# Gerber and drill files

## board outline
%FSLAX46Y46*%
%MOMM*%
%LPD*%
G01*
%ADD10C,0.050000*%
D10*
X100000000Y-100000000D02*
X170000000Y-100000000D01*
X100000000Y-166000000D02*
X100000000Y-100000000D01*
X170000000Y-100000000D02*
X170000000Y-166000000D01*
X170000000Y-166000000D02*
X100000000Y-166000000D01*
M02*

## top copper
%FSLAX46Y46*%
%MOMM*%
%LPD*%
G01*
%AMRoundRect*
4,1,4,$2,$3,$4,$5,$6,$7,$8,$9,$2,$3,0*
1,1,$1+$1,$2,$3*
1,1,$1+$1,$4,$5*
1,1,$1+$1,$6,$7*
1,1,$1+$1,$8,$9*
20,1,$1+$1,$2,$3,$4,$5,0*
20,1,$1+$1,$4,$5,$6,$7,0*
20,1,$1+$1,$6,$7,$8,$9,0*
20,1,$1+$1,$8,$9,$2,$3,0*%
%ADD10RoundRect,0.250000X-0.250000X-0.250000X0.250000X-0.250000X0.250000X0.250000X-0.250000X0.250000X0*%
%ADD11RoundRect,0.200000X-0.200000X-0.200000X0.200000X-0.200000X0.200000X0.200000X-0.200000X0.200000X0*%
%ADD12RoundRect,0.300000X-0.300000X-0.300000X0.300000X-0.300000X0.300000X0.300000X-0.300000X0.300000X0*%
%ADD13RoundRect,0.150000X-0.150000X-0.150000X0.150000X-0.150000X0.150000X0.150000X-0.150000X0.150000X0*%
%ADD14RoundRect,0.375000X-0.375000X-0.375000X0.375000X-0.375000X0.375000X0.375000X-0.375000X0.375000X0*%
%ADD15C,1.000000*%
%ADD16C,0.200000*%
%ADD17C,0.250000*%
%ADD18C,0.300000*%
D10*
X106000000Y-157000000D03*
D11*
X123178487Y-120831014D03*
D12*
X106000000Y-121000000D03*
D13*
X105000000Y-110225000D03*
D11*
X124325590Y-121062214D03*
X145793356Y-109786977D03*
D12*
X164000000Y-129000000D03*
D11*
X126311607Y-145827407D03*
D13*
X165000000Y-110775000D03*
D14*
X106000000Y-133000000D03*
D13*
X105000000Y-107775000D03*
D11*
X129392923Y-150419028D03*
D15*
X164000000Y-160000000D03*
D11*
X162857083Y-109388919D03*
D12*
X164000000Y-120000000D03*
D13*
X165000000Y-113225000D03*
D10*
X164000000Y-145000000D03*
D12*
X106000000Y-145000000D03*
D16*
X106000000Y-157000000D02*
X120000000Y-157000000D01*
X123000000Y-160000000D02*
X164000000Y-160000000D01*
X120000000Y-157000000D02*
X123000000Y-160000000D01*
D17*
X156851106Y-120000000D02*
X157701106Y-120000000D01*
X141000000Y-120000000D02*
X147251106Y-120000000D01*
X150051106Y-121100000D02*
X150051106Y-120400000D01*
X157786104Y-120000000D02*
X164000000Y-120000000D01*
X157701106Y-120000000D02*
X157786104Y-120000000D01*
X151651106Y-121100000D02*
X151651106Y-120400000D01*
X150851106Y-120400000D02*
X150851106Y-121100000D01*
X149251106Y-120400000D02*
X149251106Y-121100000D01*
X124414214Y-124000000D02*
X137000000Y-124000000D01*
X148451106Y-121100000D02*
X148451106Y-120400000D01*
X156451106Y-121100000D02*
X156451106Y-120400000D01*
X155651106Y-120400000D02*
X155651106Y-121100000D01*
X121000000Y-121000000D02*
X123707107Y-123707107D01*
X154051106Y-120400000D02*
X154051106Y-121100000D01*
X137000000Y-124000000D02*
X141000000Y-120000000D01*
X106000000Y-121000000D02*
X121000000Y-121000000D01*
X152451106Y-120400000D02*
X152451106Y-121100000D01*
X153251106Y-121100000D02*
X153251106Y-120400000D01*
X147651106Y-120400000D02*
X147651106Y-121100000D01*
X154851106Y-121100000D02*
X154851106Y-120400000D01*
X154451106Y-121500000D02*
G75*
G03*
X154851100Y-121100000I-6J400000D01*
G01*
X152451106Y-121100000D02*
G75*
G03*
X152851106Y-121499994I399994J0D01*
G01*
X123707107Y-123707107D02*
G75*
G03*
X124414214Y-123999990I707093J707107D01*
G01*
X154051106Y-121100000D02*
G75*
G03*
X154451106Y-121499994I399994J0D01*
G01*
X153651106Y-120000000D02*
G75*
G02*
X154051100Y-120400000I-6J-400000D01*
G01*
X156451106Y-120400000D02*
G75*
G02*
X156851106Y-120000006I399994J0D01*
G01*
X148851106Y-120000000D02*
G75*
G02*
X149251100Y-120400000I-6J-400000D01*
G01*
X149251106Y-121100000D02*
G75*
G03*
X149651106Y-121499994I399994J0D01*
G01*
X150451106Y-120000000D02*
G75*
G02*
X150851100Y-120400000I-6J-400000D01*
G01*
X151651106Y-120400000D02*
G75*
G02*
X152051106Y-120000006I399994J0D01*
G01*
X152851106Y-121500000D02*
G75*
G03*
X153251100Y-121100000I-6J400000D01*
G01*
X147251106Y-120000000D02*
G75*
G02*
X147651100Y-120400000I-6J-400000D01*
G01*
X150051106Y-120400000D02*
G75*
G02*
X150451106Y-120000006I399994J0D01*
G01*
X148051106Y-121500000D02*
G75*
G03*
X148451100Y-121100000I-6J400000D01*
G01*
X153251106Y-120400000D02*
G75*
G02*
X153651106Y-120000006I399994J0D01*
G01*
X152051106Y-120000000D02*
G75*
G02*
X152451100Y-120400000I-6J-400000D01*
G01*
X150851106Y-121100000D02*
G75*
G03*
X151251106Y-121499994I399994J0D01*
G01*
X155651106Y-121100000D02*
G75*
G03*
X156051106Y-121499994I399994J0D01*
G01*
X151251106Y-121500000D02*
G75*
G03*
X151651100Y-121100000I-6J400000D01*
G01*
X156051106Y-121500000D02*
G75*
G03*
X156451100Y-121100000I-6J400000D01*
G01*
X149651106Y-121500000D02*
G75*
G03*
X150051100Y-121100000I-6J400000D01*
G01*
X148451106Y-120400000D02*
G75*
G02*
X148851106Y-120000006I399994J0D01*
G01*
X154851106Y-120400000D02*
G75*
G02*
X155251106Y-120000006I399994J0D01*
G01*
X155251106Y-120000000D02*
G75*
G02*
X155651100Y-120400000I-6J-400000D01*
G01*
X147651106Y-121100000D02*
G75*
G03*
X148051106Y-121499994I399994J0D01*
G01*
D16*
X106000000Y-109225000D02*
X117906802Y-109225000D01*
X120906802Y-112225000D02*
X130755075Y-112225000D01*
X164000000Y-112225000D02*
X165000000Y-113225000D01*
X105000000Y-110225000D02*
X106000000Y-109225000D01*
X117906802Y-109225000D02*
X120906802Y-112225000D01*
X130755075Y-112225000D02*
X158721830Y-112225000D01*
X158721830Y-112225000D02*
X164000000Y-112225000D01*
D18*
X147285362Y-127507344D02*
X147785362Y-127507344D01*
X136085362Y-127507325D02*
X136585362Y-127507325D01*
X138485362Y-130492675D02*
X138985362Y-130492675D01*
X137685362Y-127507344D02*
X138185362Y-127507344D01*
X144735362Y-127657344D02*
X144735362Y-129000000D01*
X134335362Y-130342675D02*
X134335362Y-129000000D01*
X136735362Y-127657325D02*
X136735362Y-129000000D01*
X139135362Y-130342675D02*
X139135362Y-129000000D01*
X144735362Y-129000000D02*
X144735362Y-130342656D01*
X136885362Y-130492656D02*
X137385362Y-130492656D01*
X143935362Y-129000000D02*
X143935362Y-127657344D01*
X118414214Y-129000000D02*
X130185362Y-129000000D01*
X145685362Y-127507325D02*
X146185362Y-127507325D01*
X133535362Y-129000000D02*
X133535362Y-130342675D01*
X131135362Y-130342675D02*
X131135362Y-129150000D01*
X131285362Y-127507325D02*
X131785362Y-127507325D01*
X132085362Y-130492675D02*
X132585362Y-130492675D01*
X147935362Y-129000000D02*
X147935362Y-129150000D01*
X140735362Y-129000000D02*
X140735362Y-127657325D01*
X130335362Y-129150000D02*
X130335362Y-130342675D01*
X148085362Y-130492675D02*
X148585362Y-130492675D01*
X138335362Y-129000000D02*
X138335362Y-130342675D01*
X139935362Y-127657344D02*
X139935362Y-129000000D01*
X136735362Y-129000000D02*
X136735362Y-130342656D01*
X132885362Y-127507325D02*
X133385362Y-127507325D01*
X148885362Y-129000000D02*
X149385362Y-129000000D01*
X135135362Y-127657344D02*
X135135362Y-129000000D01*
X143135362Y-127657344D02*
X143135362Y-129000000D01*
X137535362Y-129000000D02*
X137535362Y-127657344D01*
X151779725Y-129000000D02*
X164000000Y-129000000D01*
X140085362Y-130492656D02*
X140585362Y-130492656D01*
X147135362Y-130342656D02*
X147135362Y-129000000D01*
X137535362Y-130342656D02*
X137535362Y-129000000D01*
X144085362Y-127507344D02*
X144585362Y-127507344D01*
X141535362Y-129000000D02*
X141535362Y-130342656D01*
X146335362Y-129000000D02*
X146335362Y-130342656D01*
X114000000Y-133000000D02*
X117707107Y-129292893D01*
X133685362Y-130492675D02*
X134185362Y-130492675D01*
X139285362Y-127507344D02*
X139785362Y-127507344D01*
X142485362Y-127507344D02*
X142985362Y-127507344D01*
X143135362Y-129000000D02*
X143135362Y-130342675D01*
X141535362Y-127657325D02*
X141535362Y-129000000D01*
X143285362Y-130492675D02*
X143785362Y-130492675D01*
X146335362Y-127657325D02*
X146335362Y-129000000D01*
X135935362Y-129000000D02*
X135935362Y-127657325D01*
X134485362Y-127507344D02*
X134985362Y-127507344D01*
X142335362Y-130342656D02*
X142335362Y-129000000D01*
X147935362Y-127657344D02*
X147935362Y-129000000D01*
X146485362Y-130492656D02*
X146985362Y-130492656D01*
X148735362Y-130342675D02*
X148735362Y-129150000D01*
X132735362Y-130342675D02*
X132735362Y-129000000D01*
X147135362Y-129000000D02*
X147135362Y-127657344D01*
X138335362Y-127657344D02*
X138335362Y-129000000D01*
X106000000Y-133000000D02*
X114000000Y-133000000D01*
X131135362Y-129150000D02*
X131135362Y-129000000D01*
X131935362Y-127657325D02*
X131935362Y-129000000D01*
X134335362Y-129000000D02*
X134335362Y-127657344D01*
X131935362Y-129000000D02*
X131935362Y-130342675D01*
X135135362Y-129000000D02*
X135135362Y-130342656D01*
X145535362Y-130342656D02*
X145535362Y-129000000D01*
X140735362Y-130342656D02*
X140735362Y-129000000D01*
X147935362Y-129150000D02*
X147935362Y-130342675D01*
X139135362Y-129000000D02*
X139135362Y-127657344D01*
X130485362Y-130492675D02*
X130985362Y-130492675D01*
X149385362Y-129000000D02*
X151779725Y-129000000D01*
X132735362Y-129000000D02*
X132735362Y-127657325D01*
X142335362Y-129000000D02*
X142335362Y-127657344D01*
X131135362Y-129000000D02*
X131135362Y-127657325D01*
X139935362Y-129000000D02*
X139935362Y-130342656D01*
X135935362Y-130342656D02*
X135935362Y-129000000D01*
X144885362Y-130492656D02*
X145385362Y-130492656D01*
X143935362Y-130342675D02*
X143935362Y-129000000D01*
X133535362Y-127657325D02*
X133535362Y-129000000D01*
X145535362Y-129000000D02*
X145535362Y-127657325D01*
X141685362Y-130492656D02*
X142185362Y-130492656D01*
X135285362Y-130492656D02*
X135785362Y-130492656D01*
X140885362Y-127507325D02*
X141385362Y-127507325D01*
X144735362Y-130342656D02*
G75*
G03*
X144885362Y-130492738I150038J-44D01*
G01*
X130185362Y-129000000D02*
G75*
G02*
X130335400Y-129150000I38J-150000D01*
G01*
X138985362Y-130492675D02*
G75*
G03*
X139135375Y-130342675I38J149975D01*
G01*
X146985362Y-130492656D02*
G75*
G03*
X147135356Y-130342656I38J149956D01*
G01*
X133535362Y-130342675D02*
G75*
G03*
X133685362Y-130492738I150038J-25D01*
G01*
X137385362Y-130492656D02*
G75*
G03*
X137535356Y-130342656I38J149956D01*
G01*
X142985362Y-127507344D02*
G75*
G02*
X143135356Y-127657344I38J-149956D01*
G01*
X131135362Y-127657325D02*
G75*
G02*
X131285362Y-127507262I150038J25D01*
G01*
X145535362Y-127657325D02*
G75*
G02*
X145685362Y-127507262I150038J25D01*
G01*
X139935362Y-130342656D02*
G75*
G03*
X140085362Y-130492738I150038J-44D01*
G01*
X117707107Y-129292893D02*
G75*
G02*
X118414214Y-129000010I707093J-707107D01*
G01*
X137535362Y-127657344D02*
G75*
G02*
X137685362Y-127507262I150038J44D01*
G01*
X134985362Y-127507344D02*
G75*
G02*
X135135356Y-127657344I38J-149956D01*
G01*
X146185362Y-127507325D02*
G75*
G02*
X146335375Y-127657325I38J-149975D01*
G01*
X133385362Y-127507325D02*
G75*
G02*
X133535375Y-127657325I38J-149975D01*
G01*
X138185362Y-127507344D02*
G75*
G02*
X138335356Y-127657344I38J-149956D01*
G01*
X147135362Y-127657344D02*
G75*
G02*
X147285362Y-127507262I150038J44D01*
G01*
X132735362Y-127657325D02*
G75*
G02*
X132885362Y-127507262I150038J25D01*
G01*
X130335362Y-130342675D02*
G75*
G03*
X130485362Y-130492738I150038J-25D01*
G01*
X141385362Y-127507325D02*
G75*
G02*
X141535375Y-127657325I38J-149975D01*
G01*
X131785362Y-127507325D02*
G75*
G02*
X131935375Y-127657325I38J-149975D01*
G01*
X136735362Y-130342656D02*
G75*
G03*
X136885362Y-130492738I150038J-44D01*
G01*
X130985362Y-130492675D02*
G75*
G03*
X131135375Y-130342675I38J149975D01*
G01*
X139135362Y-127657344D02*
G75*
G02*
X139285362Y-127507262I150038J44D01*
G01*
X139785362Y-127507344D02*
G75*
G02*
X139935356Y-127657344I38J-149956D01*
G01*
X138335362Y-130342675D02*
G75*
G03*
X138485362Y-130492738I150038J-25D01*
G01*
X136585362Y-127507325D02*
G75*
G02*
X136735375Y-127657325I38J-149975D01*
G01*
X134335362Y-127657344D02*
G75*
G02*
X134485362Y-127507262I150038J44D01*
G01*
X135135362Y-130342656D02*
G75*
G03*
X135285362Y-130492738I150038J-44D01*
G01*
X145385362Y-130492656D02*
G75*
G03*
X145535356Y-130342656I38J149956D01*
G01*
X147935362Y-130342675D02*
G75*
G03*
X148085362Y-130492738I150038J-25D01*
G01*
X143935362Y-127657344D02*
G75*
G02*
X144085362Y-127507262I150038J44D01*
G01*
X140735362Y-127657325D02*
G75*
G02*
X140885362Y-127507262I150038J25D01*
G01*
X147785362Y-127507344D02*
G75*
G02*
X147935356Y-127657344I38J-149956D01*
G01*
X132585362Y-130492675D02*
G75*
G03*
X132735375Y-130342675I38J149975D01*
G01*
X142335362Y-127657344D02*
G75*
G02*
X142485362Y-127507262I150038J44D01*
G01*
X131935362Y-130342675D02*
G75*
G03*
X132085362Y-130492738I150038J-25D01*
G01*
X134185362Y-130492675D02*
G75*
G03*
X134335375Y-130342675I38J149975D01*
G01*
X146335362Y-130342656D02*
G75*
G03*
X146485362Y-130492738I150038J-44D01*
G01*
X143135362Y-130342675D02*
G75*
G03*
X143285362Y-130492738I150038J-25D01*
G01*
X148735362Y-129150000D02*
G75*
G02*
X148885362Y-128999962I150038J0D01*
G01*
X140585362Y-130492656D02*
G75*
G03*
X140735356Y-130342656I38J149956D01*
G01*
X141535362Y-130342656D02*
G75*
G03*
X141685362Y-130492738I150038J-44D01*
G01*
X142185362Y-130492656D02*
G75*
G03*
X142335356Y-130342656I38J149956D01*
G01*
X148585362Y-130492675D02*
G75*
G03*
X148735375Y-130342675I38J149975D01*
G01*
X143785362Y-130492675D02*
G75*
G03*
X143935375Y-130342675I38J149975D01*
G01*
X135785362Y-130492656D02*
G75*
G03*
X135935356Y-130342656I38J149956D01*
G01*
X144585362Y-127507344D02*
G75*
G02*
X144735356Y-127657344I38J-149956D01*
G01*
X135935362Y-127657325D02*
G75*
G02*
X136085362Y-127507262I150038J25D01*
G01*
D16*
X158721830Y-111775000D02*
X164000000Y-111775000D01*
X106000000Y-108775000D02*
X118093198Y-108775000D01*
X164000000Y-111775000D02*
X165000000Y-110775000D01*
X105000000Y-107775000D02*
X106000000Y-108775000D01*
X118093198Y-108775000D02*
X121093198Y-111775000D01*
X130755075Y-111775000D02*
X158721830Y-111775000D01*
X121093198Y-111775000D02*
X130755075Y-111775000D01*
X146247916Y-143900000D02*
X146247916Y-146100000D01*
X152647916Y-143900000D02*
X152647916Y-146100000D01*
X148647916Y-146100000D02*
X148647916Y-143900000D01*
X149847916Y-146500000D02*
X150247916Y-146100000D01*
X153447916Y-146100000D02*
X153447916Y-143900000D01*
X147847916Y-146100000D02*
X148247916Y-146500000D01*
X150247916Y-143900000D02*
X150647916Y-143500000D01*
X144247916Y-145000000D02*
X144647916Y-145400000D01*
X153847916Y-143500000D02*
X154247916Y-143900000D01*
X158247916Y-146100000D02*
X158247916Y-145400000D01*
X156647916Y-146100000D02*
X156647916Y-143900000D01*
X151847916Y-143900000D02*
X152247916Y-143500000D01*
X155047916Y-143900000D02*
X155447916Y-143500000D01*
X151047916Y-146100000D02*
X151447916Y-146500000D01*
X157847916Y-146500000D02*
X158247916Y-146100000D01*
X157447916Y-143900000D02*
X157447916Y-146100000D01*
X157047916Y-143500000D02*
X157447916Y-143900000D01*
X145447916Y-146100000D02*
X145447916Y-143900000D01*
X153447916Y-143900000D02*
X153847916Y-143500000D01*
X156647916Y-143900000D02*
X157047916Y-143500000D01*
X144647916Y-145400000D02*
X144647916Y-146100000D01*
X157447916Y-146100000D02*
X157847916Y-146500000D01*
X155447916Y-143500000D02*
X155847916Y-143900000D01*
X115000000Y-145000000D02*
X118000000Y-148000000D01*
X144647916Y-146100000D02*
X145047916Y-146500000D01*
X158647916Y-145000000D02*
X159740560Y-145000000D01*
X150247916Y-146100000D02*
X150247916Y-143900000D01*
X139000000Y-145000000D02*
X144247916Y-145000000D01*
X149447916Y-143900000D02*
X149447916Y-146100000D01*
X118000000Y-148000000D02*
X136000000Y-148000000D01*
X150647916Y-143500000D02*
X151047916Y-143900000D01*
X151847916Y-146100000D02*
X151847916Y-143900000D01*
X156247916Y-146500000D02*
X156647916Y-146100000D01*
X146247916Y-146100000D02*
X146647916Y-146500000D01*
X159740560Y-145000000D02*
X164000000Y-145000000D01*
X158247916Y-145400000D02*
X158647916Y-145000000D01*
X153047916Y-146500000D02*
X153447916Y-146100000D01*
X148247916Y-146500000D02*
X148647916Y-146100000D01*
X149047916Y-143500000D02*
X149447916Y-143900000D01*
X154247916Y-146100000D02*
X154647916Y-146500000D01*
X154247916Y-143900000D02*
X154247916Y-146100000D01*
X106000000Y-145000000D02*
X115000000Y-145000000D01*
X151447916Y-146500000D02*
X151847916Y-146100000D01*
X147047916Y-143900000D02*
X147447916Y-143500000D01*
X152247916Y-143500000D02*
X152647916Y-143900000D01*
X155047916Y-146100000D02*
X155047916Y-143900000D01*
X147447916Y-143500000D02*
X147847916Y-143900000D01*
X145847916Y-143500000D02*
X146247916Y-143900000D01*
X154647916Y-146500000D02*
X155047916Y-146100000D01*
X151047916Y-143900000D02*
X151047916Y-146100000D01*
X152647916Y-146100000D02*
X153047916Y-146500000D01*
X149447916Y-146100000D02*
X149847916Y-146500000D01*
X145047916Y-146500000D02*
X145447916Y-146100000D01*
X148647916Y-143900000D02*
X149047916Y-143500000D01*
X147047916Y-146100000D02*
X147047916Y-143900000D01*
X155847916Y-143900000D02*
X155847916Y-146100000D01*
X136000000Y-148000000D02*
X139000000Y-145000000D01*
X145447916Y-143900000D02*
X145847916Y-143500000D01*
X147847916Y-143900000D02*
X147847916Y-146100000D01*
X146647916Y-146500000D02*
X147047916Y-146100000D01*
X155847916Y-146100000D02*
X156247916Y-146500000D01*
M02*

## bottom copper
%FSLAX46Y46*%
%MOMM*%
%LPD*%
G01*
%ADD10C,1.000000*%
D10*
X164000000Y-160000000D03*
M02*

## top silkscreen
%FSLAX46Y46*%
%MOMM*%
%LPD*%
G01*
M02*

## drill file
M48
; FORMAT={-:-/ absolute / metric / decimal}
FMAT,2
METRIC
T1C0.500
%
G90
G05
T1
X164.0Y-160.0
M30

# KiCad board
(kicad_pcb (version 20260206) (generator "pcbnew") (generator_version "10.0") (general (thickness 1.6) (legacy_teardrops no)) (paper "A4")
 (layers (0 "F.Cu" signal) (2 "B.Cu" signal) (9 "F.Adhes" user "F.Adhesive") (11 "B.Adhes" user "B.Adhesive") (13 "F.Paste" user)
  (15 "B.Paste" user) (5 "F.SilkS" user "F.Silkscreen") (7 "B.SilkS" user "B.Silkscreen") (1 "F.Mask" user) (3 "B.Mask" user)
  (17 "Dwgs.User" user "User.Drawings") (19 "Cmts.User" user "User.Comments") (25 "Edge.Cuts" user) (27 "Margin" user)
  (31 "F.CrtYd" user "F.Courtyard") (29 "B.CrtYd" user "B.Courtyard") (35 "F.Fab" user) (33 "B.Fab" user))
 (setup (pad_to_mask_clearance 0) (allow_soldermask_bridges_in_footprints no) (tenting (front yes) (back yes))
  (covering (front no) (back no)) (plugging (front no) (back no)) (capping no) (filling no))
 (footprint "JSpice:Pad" (layer "F.Cu") (at 106 157)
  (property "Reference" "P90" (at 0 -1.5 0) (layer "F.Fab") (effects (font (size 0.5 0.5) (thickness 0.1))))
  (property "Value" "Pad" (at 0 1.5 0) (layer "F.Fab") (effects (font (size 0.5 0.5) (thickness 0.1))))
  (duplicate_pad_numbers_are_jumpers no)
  (pad "1" smd roundrect (at 0 0) (size 1 1) (layers "F.Cu" "F.Mask") (roundrect_rratio 0.25) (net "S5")))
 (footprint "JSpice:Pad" (layer "F.Cu") (at 123.178487 120.831014)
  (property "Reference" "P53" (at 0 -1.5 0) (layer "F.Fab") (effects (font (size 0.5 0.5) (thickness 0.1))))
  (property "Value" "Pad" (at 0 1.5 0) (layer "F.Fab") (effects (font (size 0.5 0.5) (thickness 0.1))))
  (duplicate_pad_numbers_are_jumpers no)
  (pad "1" smd roundrect (at 0 0) (size 0.8 0.8) (layers "F.Cu" "F.Mask") (roundrect_rratio 0.25) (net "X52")))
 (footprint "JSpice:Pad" (layer "F.Cu") (at 106 121)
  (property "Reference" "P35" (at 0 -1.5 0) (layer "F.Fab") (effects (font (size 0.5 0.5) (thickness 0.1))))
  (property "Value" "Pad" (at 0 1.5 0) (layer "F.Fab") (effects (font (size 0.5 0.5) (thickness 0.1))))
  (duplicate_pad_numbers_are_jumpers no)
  (pad "1" smd roundrect (at 0 0) (size 1.2 1.2) (layers "F.Cu" "F.Mask") (roundrect_rratio 0.25) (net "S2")))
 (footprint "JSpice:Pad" (layer "F.Cu") (at 105 110.225)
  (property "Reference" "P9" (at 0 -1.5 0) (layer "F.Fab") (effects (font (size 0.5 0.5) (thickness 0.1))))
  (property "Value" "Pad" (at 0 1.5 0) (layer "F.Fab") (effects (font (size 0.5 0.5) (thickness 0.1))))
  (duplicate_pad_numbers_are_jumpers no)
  (pad "1" smd roundrect (at 0 0) (size 0.6 0.6) (layers "F.Cu" "F.Mask") (roundrect_rratio 0.25) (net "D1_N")))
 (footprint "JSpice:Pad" (layer "F.Cu") (at 124.32559 121.062214)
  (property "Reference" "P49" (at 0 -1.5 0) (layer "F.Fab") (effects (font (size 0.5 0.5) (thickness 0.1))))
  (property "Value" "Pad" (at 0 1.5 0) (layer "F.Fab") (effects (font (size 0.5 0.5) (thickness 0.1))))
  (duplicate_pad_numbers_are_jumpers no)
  (pad "1" smd roundrect (at 0 0) (size 0.8 0.8) (layers "F.Cu" "F.Mask") (roundrect_rratio 0.25) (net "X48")))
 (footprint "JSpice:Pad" (layer "F.Cu") (at 145.793356 109.786977)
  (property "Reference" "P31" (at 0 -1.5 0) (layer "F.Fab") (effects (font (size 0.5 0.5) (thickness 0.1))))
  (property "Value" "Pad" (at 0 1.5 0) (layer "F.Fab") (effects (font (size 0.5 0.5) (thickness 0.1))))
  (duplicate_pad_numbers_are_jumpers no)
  (pad "1" smd roundrect (at 0 0) (size 0.8 0.8) (layers "F.Cu" "F.Mask") (roundrect_rratio 0.25) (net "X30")))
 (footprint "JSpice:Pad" (layer "F.Cu") (at 164 129)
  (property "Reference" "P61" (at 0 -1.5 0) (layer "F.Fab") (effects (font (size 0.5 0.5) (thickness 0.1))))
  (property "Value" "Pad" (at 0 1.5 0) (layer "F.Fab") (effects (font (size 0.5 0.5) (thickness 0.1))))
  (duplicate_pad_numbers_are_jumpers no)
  (pad "1" smd roundrect (at 0 0) (size 1.2 1.2) (layers "F.Cu" "F.Mask") (roundrect_rratio 0.25) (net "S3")))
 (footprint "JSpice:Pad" (layer "F.Cu") (at 126.311607 145.827407)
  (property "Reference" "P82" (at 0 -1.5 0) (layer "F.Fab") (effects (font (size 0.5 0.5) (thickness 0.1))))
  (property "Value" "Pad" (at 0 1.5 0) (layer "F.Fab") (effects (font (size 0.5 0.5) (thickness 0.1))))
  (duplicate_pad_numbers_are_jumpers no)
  (pad "1" smd roundrect (at 0 0) (size 0.8 0.8) (layers "F.Cu" "F.Mask") (roundrect_rratio 0.25) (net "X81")))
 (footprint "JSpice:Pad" (layer "F.Cu") (at 165 110.775)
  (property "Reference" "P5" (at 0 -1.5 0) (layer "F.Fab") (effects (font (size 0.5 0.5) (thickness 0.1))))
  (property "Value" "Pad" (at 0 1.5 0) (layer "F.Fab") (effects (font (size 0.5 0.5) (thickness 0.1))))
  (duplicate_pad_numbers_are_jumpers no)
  (pad "1" smd roundrect (at 0 0) (size 0.6 0.6) (layers "F.Cu" "F.Mask") (roundrect_rratio 0.25) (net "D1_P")))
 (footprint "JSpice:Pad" (layer "F.Cu") (at 106 133)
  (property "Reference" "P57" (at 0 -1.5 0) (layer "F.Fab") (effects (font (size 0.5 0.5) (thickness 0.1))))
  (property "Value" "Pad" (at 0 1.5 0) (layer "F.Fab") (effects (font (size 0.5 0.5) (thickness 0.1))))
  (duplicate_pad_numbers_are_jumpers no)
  (pad "1" smd roundrect (at 0 0) (size 1.5 1.5) (layers "F.Cu" "F.Mask") (roundrect_rratio 0.25) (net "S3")))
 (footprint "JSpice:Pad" (layer "F.Cu") (at 105 107.775)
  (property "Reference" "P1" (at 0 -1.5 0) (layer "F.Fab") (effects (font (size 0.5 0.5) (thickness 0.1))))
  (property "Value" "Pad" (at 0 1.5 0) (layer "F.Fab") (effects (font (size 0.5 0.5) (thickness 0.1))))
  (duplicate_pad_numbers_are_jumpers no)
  (pad "1" smd roundrect (at 0 0) (size 0.6 0.6) (layers "F.Cu" "F.Mask") (roundrect_rratio 0.25) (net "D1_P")))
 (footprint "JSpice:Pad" (layer "F.Cu") (at 129.392923 150.419028)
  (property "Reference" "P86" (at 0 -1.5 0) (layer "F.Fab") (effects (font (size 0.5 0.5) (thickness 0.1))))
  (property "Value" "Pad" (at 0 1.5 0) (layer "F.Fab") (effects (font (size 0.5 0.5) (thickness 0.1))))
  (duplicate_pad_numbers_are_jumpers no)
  (pad "1" smd roundrect (at 0 0) (size 0.8 0.8) (layers "F.Cu" "F.Mask") (roundrect_rratio 0.25) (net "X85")))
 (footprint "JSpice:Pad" (layer "F.Cu") (at 164 160)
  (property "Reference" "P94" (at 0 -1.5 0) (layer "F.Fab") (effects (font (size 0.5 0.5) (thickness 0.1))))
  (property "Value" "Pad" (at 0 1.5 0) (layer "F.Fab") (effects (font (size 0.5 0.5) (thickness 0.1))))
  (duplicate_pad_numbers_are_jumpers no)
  (pad "1" thru_hole circle (at 0 0) (size 1 1) (drill 0.5) (layers "*.Cu" "*.Mask") (remove_unused_layers no) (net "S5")))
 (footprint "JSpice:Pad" (layer "F.Cu") (at 162.857083 109.388919)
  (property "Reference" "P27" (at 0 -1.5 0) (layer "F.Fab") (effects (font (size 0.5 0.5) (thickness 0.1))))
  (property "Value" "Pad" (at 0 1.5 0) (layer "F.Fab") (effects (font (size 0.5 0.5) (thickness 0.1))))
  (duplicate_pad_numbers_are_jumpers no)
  (pad "1" smd roundrect (at 0 0) (size 0.8 0.8) (layers "F.Cu" "F.Mask") (roundrect_rratio 0.25) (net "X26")))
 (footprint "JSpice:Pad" (layer "F.Cu") (at 164 120)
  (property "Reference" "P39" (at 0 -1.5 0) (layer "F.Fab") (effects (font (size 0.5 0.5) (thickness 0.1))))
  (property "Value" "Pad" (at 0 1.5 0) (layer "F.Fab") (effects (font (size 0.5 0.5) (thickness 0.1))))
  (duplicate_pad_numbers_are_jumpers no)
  (pad "1" smd roundrect (at 0 0) (size 1.2 1.2) (layers "F.Cu" "F.Mask") (roundrect_rratio 0.25) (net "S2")))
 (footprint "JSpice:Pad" (layer "F.Cu") (at 165 113.225)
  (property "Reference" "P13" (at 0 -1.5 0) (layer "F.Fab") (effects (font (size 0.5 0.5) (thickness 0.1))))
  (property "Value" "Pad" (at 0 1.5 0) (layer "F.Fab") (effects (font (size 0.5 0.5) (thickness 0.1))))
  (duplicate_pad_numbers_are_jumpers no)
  (pad "1" smd roundrect (at 0 0) (size 0.6 0.6) (layers "F.Cu" "F.Mask") (roundrect_rratio 0.25) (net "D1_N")))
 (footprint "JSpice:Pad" (layer "F.Cu") (at 164 145)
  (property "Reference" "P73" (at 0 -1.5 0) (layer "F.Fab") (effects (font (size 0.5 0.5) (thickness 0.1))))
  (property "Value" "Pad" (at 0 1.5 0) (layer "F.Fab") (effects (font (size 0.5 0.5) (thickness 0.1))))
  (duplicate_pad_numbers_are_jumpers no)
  (pad "1" smd roundrect (at 0 0) (size 1 1) (layers "F.Cu" "F.Mask") (roundrect_rratio 0.25) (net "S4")))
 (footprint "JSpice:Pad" (layer "F.Cu") (at 106 145)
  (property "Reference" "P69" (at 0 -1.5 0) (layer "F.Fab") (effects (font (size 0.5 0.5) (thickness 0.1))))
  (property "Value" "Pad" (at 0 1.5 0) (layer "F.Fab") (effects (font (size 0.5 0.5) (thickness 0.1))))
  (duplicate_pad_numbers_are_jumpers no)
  (pad "1" smd roundrect (at 0 0) (size 1.2 1.2) (layers "F.Cu" "F.Mask") (roundrect_rratio 0.25) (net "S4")))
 (gr_line (start 100 100) (end 170 100) (stroke (width 0.05) (type default)) (layer "Edge.Cuts"))
 (gr_line (start 100 166) (end 100 100) (stroke (width 0.05) (type default)) (layer "Edge.Cuts"))
 (gr_line (start 170 100) (end 170 166) (stroke (width 0.05) (type default)) (layer "Edge.Cuts"))
 (gr_line (start 170 166) (end 100 166) (stroke (width 0.05) (type default)) (layer "Edge.Cuts"))
 (segment (start 106 157) (end 120 157) (width 0.2) (layer "F.Cu") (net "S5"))
 (segment (start 123 160) (end 164 160) (width 0.2) (layer "F.Cu") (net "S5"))
 (segment (start 120 157) (end 123 160) (width 0.2) (layer "F.Cu") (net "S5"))
 (segment (start 156.851106 120) (end 157.701106 120) (width 0.25) (layer "F.Cu") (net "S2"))
 (segment (start 141 120) (end 147.251106 120) (width 0.25) (layer "F.Cu") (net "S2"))
 (segment (start 150.051106 121.1) (end 150.051106 120.4) (width 0.25) (layer "F.Cu") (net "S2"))
 (segment (start 157.786104 120) (end 164 120) (width 0.25) (layer "F.Cu") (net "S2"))
 (segment (start 157.701106 120) (end 157.786104 120) (width 0.25) (layer "F.Cu") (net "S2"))
 (segment (start 151.651106 121.1) (end 151.651106 120.4) (width 0.25) (layer "F.Cu") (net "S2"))
 (segment (start 150.851106 120.4) (end 150.851106 121.1) (width 0.25) (layer "F.Cu") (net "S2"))
 (segment (start 149.251106 120.4) (end 149.251106 121.1) (width 0.25) (layer "F.Cu") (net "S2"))
 (segment (start 124.414214 124) (end 137 124) (width 0.25) (layer "F.Cu") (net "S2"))
 (segment (start 148.451106 121.1) (end 148.451106 120.4) (width 0.25) (layer "F.Cu") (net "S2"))
 (segment (start 156.451106 121.1) (end 156.451106 120.4) (width 0.25) (layer "F.Cu") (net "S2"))
 (segment (start 155.651106 120.4) (end 155.651106 121.1) (width 0.25) (layer "F.Cu") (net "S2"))
 (segment (start 121 121) (end 123.707107 123.707107) (width 0.25) (layer "F.Cu") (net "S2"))
 (segment (start 154.051106 120.4) (end 154.051106 121.1) (width 0.25) (layer "F.Cu") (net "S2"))
 (segment (start 137 124) (end 141 120) (width 0.25) (layer "F.Cu") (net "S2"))
 (segment (start 106 121) (end 121 121) (width 0.25) (layer "F.Cu") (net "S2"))
 (segment (start 152.451106 120.4) (end 152.451106 121.1) (width 0.25) (layer "F.Cu") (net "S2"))
 (segment (start 153.251106 121.1) (end 153.251106 120.4) (width 0.25) (layer "F.Cu") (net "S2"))
 (segment (start 147.651106 120.4) (end 147.651106 121.1) (width 0.25) (layer "F.Cu") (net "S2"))
 (segment (start 154.851106 121.1) (end 154.851106 120.4) (width 0.25) (layer "F.Cu") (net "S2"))
 (arc (start 154.451106 121.5) (mid 154.733949 121.382843) (end 154.851106 121.1) (width 0.25) (layer "F.Cu") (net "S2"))
 (arc (start 152.451106 121.1) (mid 152.568263 121.382843) (end 152.851106 121.5) (width 0.25) (layer "F.Cu") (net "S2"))
 (arc (start 123.707107 123.707107) (mid 124.03153 123.92388) (end 124.414214 124) (width 0.25) (layer "F.Cu") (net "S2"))
 (arc (start 154.051106 121.1) (mid 154.168263 121.382843) (end 154.451106 121.5) (width 0.25) (layer "F.Cu") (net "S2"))
 (arc (start 153.651106 120) (mid 153.933949 120.117157) (end 154.051106 120.4) (width 0.25) (layer "F.Cu") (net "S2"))
 (arc (start 156.451106 120.4) (mid 156.568263 120.117157) (end 156.851106 120) (width 0.25) (layer "F.Cu") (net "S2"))
 (arc (start 148.851106 120) (mid 149.133949 120.117157) (end 149.251106 120.4) (width 0.25) (layer "F.Cu") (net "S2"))
 (arc (start 149.251106 121.1) (mid 149.368263 121.382843) (end 149.651106 121.5) (width 0.25) (layer "F.Cu") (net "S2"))
 (arc (start 150.451106 120) (mid 150.733949 120.117157) (end 150.851106 120.4) (width 0.25) (layer "F.Cu") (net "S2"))
 (arc (start 151.651106 120.4) (mid 151.768263 120.117157) (end 152.051106 120) (width 0.25) (layer "F.Cu") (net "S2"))
 (arc (start 152.851106 121.5) (mid 153.133949 121.382843) (end 153.251106 121.1) (width 0.25) (layer "F.Cu") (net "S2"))
 (arc (start 147.251106 120) (mid 147.533949 120.117157) (end 147.651106 120.4) (width 0.25) (layer "F.Cu") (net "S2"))
 (arc (start 150.051106 120.4) (mid 150.168263 120.117157) (end 150.451106 120) (width 0.25) (layer "F.Cu") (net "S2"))
 (arc (start 148.051106 121.5) (mid 148.333949 121.382843) (end 148.451106 121.1) (width 0.25) (layer "F.Cu") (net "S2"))
 (arc (start 153.251106 120.4) (mid 153.368263 120.117157) (end 153.651106 120) (width 0.25) (layer "F.Cu") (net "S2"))
 (arc (start 152.051106 120) (mid 152.333949 120.117157) (end 152.451106 120.4) (width 0.25) (layer "F.Cu") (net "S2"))
 (arc (start 150.851106 121.1) (mid 150.968263 121.382843) (end 151.251106 121.5) (width 0.25) (layer "F.Cu") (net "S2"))
 (arc (start 155.651106 121.1) (mid 155.768263 121.382843) (end 156.051106 121.5) (width 0.25) (layer "F.Cu") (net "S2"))
 (arc (start 151.251106 121.5) (mid 151.533949 121.382843) (end 151.651106 121.1) (width 0.25) (layer "F.Cu") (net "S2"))
 (arc (start 156.051106 121.5) (mid 156.333949 121.382843) (end 156.451106 121.1) (width 0.25) (layer "F.Cu") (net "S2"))
 (arc (start 149.651106 121.5) (mid 149.933949 121.382843) (end 150.051106 121.1) (width 0.25) (layer "F.Cu") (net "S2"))
 (arc (start 148.451106 120.4) (mid 148.568263 120.117157) (end 148.851106 120) (width 0.25) (layer "F.Cu") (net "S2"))
 (arc (start 154.851106 120.4) (mid 154.968263 120.117157) (end 155.251106 120) (width 0.25) (layer "F.Cu") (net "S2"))
 (arc (start 155.251106 120) (mid 155.533949 120.117157) (end 155.651106 120.4) (width 0.25) (layer "F.Cu") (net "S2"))
 (arc (start 147.651106 121.1) (mid 147.768263 121.382843) (end 148.051106 121.5) (width 0.25) (layer "F.Cu") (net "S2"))
 (segment (start 106 109.225) (end 117.906802 109.225) (width 0.2) (layer "F.Cu") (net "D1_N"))
 (segment (start 120.906802 112.225) (end 130.755075 112.225) (width 0.2) (layer "F.Cu") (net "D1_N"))
 (segment (start 164 112.225) (end 165 113.225) (width 0.2) (layer "F.Cu") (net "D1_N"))
 (segment (start 105 110.225) (end 106 109.225) (width 0.2) (layer "F.Cu") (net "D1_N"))
 (segment (start 117.906802 109.225) (end 120.906802 112.225) (width 0.2) (layer "F.Cu") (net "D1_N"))
 (segment (start 130.755075 112.225) (end 158.72183 112.225) (width 0.2) (layer "F.Cu") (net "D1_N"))
 (segment (start 158.72183 112.225) (end 164 112.225) (width 0.2) (layer "F.Cu") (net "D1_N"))
 (segment (start 147.285362 127.507344) (end 147.785362 127.507344) (width 0.3) (layer "F.Cu") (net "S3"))
 (segment (start 136.085362 127.507325) (end 136.585362 127.507325) (width 0.3) (layer "F.Cu") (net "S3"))
 (segment (start 138.485362 130.492675) (end 138.985362 130.492675) (width 0.3) (layer "F.Cu") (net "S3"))
 (segment (start 137.685362 127.507344) (end 138.185362 127.507344) (width 0.3) (layer "F.Cu") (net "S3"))
 (segment (start 144.735362 127.657344) (end 144.735362 129) (width 0.3) (layer "F.Cu") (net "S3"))
 (segment (start 134.335362 130.342675) (end 134.335362 129) (width 0.3) (layer "F.Cu") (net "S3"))
 (segment (start 136.735362 127.657325) (end 136.735362 129) (width 0.3) (layer "F.Cu") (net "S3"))
 (segment (start 139.135362 130.342675) (end 139.135362 129) (width 0.3) (layer "F.Cu") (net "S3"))
 (segment (start 144.735362 129) (end 144.735362 130.342656) (width 0.3) (layer "F.Cu") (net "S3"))
 (segment (start 136.885362 130.492656) (end 137.385362 130.492656) (width 0.3) (layer "F.Cu") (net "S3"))
 (segment (start 143.935362 129) (end 143.935362 127.657344) (width 0.3) (layer "F.Cu") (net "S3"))
 (segment (start 118.414214 129) (end 130.185362 129) (width 0.3) (layer "F.Cu") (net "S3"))
 (segment (start 145.685362 127.507325) (end 146.185362 127.507325) (width 0.3) (layer "F.Cu") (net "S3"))
 (segment (start 133.535362 129) (end 133.535362 130.342675) (width 0.3) (layer "F.Cu") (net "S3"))
 (segment (start 131.135362 130.342675) (end 131.135362 129.15) (width 0.3) (layer "F.Cu") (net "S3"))
 (segment (start 131.285362 127.507325) (end 131.785362 127.507325) (width 0.3) (layer "F.Cu") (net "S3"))
 (segment (start 132.085362 130.492675) (end 132.585362 130.492675) (width 0.3) (layer "F.Cu") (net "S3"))
 (segment (start 147.935362 129) (end 147.935362 129.15) (width 0.3) (layer "F.Cu") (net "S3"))
 (segment (start 140.735362 129) (end 140.735362 127.657325) (width 0.3) (layer "F.Cu") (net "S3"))
 (segment (start 130.335362 129.15) (end 130.335362 130.342675) (width 0.3) (layer "F.Cu") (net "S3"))
 (segment (start 148.085362 130.492675) (end 148.585362 130.492675) (width 0.3) (layer "F.Cu") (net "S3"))
 (segment (start 138.335362 129) (end 138.335362 130.342675) (width 0.3) (layer "F.Cu") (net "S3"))
 (segment (start 139.935362 127.657344) (end 139.935362 129) (width 0.3) (layer "F.Cu") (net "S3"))
 (segment (start 136.735362 129) (end 136.735362 130.342656) (width 0.3) (layer "F.Cu") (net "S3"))
 (segment (start 132.885362 127.507325) (end 133.385362 127.507325) (width 0.3) (layer "F.Cu") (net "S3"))
 (segment (start 148.885362 129) (end 149.385362 129) (width 0.3) (layer "F.Cu") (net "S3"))
 (segment (start 135.135362 127.657344) (end 135.135362 129) (width 0.3) (layer "F.Cu") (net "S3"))
 (segment (start 143.135362 127.657344) (end 143.135362 129) (width 0.3) (layer "F.Cu") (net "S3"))
 (segment (start 137.535362 129) (end 137.535362 127.657344) (width 0.3) (layer "F.Cu") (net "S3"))
 (segment (start 151.779725 129) (end 164 129) (width 0.3) (layer "F.Cu") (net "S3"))
 (segment (start 140.085362 130.492656) (end 140.585362 130.492656) (width 0.3) (layer "F.Cu") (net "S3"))
 (segment (start 147.135362 130.342656) (end 147.135362 129) (width 0.3) (layer "F.Cu") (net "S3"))
 (segment (start 137.535362 130.342656) (end 137.535362 129) (width 0.3) (layer "F.Cu") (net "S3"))
 (segment (start 144.085362 127.507344) (end 144.585362 127.507344) (width 0.3) (layer "F.Cu") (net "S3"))
 (segment (start 141.535362 129) (end 141.535362 130.342656) (width 0.3) (layer "F.Cu") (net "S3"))
 (segment (start 146.335362 129) (end 146.335362 130.342656) (width 0.3) (layer "F.Cu") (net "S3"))
 (segment (start 114 133) (end 117.707107 129.292893) (width 0.3) (layer "F.Cu") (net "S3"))
 (segment (start 133.685362 130.492675) (end 134.185362 130.492675) (width 0.3) (layer "F.Cu") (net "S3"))
 (segment (start 139.285362 127.507344) (end 139.785362 127.507344) (width 0.3) (layer "F.Cu") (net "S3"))
 (segment (start 142.485362 127.507344) (end 142.985362 127.507344) (width 0.3) (layer "F.Cu") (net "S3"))
 (segment (start 143.135362 129) (end 143.135362 130.342675) (width 0.3) (layer "F.Cu") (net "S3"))
 (segment (start 141.535362 127.657325) (end 141.535362 129) (width 0.3) (layer "F.Cu") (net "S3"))
 (segment (start 143.285362 130.492675) (end 143.785362 130.492675) (width 0.3) (layer "F.Cu") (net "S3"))
 (segment (start 146.335362 127.657325) (end 146.335362 129) (width 0.3) (layer "F.Cu") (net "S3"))
 (segment (start 135.935362 129) (end 135.935362 127.657325) (width 0.3) (layer "F.Cu") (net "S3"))
 (segment (start 134.485362 127.507344) (end 134.985362 127.507344) (width 0.3) (layer "F.Cu") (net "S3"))
 (segment (start 142.335362 130.342656) (end 142.335362 129) (width 0.3) (layer "F.Cu") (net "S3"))
 (segment (start 147.935362 127.657344) (end 147.935362 129) (width 0.3) (layer "F.Cu") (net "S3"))
 (segment (start 146.485362 130.492656) (end 146.985362 130.492656) (width 0.3) (layer "F.Cu") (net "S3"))
 (segment (start 148.735362 130.342675) (end 148.735362 129.15) (width 0.3) (layer "F.Cu") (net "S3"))
 (segment (start 132.735362 130.342675) (end 132.735362 129) (width 0.3) (layer "F.Cu") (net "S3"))
 (segment (start 147.135362 129) (end 147.135362 127.657344) (width 0.3) (layer "F.Cu") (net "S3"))
 (segment (start 138.335362 127.657344) (end 138.335362 129) (width 0.3) (layer "F.Cu") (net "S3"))
 (segment (start 106 133) (end 114 133) (width 0.3) (layer "F.Cu") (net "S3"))
 (segment (start 131.135362 129.15) (end 131.135362 129) (width 0.3) (layer "F.Cu") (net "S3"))
 (segment (start 131.935362 127.657325) (end 131.935362 129) (width 0.3) (layer "F.Cu") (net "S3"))
 (segment (start 134.335362 129) (end 134.335362 127.657344) (width 0.3) (layer "F.Cu") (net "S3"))
 (segment (start 131.935362 129) (end 131.935362 130.342675) (width 0.3) (layer "F.Cu") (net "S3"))
 (segment (start 135.135362 129) (end 135.135362 130.342656) (width 0.3) (layer "F.Cu") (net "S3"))
 (segment (start 145.535362 130.342656) (end 145.535362 129) (width 0.3) (layer "F.Cu") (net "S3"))
 (segment (start 140.735362 130.342656) (end 140.735362 129) (width 0.3) (layer "F.Cu") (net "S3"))
 (segment (start 147.935362 129.15) (end 147.935362 130.342675) (width 0.3) (layer "F.Cu") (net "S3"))
 (segment (start 139.135362 129) (end 139.135362 127.657344) (width 0.3) (layer "F.Cu") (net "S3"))
 (segment (start 130.485362 130.492675) (end 130.985362 130.492675) (width 0.3) (layer "F.Cu") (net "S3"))
 (segment (start 149.385362 129) (end 151.779725 129) (width 0.3) (layer "F.Cu") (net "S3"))
 (segment (start 132.735362 129) (end 132.735362 127.657325) (width 0.3) (layer "F.Cu") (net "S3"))
 (segment (start 142.335362 129) (end 142.335362 127.657344) (width 0.3) (layer "F.Cu") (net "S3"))
 (segment (start 131.135362 129) (end 131.135362 127.657325) (width 0.3) (layer "F.Cu") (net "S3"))
 (segment (start 139.935362 129) (end 139.935362 130.342656) (width 0.3) (layer "F.Cu") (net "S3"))
 (segment (start 135.935362 130.342656) (end 135.935362 129) (width 0.3) (layer "F.Cu") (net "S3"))
 (segment (start 144.885362 130.492656) (end 145.385362 130.492656) (width 0.3) (layer "F.Cu") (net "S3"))
 (segment (start 143.935362 130.342675) (end 143.935362 129) (width 0.3) (layer "F.Cu") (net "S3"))
 (segment (start 133.535362 127.657325) (end 133.535362 129) (width 0.3) (layer "F.Cu") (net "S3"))
 (segment (start 145.535362 129) (end 145.535362 127.657325) (width 0.3) (layer "F.Cu") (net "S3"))
 (segment (start 141.685362 130.492656) (end 142.185362 130.492656) (width 0.3) (layer "F.Cu") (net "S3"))
 (segment (start 135.285362 130.492656) (end 135.785362 130.492656) (width 0.3) (layer "F.Cu") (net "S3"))
 (segment (start 140.885362 127.507325) (end 141.385362 127.507325) (width 0.3) (layer "F.Cu") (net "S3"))
 (arc (start 144.735362 130.342656) (mid 144.779296 130.448722) (end 144.885362 130.492656) (width 0.3) (layer "F.Cu") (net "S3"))
 (arc (start 130.185362 129) (mid 130.291428 129.043934) (end 130.335362 129.15) (width 0.3) (layer "F.Cu") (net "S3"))
 (arc (start 138.985362 130.492675) (mid 139.091428 130.448741) (end 139.135362 130.342675) (width 0.3) (layer "F.Cu") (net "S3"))
 (arc (start 146.985362 130.492656) (mid 147.091428 130.448722) (end 147.135362 130.342656) (width 0.3) (layer "F.Cu") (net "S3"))
 (arc (start 133.535362 130.342675) (mid 133.579296 130.448741) (end 133.685362 130.492675) (width 0.3) (layer "F.Cu") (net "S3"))
 (arc (start 137.385362 130.492656) (mid 137.491428 130.448722) (end 137.535362 130.342656) (width 0.3) (layer "F.Cu") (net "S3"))
 (arc (start 142.985362 127.507344) (mid 143.091428 127.551278) (end 143.135362 127.657344) (width 0.3) (layer "F.Cu") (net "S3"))
 (arc (start 131.135362 127.657325) (mid 131.179296 127.551259) (end 131.285362 127.507325) (width 0.3) (layer "F.Cu") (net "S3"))
 (arc (start 145.535362 127.657325) (mid 145.579296 127.551259) (end 145.685362 127.507325) (width 0.3) (layer "F.Cu") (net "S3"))
 (arc (start 139.935362 130.342656) (mid 139.979296 130.448722) (end 140.085362 130.492656) (width 0.3) (layer "F.Cu") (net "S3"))
 (arc (start 117.707107 129.292893) (mid 118.03153 129.07612) (end 118.414214 129) (width 0.3) (layer "F.Cu") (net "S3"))
 (arc (start 137.535362 127.657344) (mid 137.579296 127.551278) (end 137.685362 127.507344) (width 0.3) (layer "F.Cu") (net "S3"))
 (arc (start 134.985362 127.507344) (mid 135.091428 127.551278) (end 135.135362 127.657344) (width 0.3) (layer "F.Cu") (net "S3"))
 (arc (start 146.185362 127.507325) (mid 146.291428 127.551259) (end 146.335362 127.657325) (width 0.3) (layer "F.Cu") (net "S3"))
 (arc (start 133.385362 127.507325) (mid 133.491428 127.551259) (end 133.535362 127.657325) (width 0.3) (layer "F.Cu") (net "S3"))
 (arc (start 138.185362 127.507344) (mid 138.291428 127.551278) (end 138.335362 127.657344) (width 0.3) (layer "F.Cu") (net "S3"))
 (arc (start 147.135362 127.657344) (mid 147.179296 127.551278) (end 147.285362 127.507344) (width 0.3) (layer "F.Cu") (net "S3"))
 (arc (start 132.735362 127.657325) (mid 132.779296 127.551259) (end 132.885362 127.507325) (width 0.3) (layer "F.Cu") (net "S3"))
 (arc (start 130.335362 130.342675) (mid 130.379296 130.448741) (end 130.485362 130.492675) (width 0.3) (layer "F.Cu") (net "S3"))
 (arc (start 141.385362 127.507325) (mid 141.491428 127.551259) (end 141.535362 127.657325) (width 0.3) (layer "F.Cu") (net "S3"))
 (arc (start 131.785362 127.507325) (mid 131.891428 127.551259) (end 131.935362 127.657325) (width 0.3) (layer "F.Cu") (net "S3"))
 (arc (start 136.735362 130.342656) (mid 136.779296 130.448722) (end 136.885362 130.492656) (width 0.3) (layer "F.Cu") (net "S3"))
 (arc (start 130.985362 130.492675) (mid 131.091428 130.448741) (end 131.135362 130.342675) (width 0.3) (layer "F.Cu") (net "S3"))
 (arc (start 139.135362 127.657344) (mid 139.179296 127.551278) (end 139.285362 127.507344) (width 0.3) (layer "F.Cu") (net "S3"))
 (arc (start 139.785362 127.507344) (mid 139.891428 127.551278) (end 139.935362 127.657344) (width 0.3) (layer "F.Cu") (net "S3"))
 (arc (start 138.335362 130.342675) (mid 138.379296 130.448741) (end 138.485362 130.492675) (width 0.3) (layer "F.Cu") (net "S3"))
 (arc (start 136.585362 127.507325) (mid 136.691428 127.551259) (end 136.735362 127.657325) (width 0.3) (layer "F.Cu") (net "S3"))
 (arc (start 134.335362 127.657344) (mid 134.379296 127.551278) (end 134.485362 127.507344) (width 0.3) (layer "F.Cu") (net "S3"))
 (arc (start 135.135362 130.342656) (mid 135.179296 130.448722) (end 135.285362 130.492656) (width 0.3) (layer "F.Cu") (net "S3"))
 (arc (start 145.385362 130.492656) (mid 145.491428 130.448722) (end 145.535362 130.342656) (width 0.3) (layer "F.Cu") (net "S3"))
 (arc (start 147.935362 130.342675) (mid 147.979296 130.448741) (end 148.085362 130.492675) (width 0.3) (layer "F.Cu") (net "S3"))
 (arc (start 143.935362 127.657344) (mid 143.979296 127.551278) (end 144.085362 127.507344) (width 0.3) (layer "F.Cu") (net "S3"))
 (arc (start 140.735362 127.657325) (mid 140.779296 127.551259) (end 140.885362 127.507325) (width 0.3) (layer "F.Cu") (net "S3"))
 (arc (start 147.785362 127.507344) (mid 147.891428 127.551278) (end 147.935362 127.657344) (width 0.3) (layer "F.Cu") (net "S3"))
 (arc (start 132.585362 130.492675) (mid 132.691428 130.448741) (end 132.735362 130.342675) (width 0.3) (layer "F.Cu") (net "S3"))
 (arc (start 142.335362 127.657344) (mid 142.379296 127.551278) (end 142.485362 127.507344) (width 0.3) (layer "F.Cu") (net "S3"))
 (arc (start 131.935362 130.342675) (mid 131.979296 130.448741) (end 132.085362 130.492675) (width 0.3) (layer "F.Cu") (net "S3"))
 (arc (start 134.185362 130.492675) (mid 134.291428 130.448741) (end 134.335362 130.342675) (width 0.3) (layer "F.Cu") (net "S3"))
 (arc (start 146.335362 130.342656) (mid 146.379296 130.448722) (end 146.485362 130.492656) (width 0.3) (layer "F.Cu") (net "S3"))
 (arc (start 143.135362 130.342675) (mid 143.179296 130.448741) (end 143.285362 130.492675) (width 0.3) (layer "F.Cu") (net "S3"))
 (arc (start 148.735362 129.15) (mid 148.779296 129.043934) (end 148.885362 129) (width 0.3) (layer "F.Cu") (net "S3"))
 (arc (start 140.585362 130.492656) (mid 140.691428 130.448722) (end 140.735362 130.342656) (width 0.3) (layer "F.Cu") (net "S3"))
 (arc (start 141.535362 130.342656) (mid 141.579296 130.448722) (end 141.685362 130.492656) (width 0.3) (layer "F.Cu") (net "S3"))
 (arc (start 142.185362 130.492656) (mid 142.291428 130.448722) (end 142.335362 130.342656) (width 0.3) (layer "F.Cu") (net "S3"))
 (arc (start 148.585362 130.492675) (mid 148.691428 130.448741) (end 148.735362 130.342675) (width 0.3) (layer "F.Cu") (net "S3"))
 (arc (start 143.785362 130.492675) (mid 143.891428 130.448741) (end 143.935362 130.342675) (width 0.3) (layer "F.Cu") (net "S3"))
 (arc (start 135.785362 130.492656) (mid 135.891428 130.448722) (end 135.935362 130.342656) (width 0.3) (layer "F.Cu") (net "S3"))
 (arc (start 144.585362 127.507344) (mid 144.691428 127.551278) (end 144.735362 127.657344) (width 0.3) (layer "F.Cu") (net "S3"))
 (arc (start 135.935362 127.657325) (mid 135.979296 127.551259) (end 136.085362 127.507325) (width 0.3) (layer "F.Cu") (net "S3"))
 (segment (start 158.72183 111.775) (end 164 111.775) (width 0.2) (layer "F.Cu") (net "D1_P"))
 (segment (start 106 108.775) (end 118.093198 108.775) (width 0.2) (layer "F.Cu") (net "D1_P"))
 (segment (start 164 111.775) (end 165 110.775) (width 0.2) (layer "F.Cu") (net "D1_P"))
 (segment (start 105 107.775) (end 106 108.775) (width 0.2) (layer "F.Cu") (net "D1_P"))
 (segment (start 118.093198 108.775) (end 121.093198 111.775) (width 0.2) (layer "F.Cu") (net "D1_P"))
 (segment (start 130.755075 111.775) (end 158.72183 111.775) (width 0.2) (layer "F.Cu") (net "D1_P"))
 (segment (start 121.093198 111.775) (end 130.755075 111.775) (width 0.2) (layer "F.Cu") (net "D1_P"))
 (segment (start 146.247916 143.9) (end 146.247916 146.1) (width 0.2) (layer "F.Cu") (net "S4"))
 (segment (start 152.647916 143.9) (end 152.647916 146.1) (width 0.2) (layer "F.Cu") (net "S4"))
 (segment (start 148.647916 146.1) (end 148.647916 143.9) (width 0.2) (layer "F.Cu") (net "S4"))
 (segment (start 149.847916 146.5) (end 150.247916 146.1) (width 0.2) (layer "F.Cu") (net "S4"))
 (segment (start 153.447916 146.1) (end 153.447916 143.9) (width 0.2) (layer "F.Cu") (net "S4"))
 (segment (start 147.847916 146.1) (end 148.247916 146.5) (width 0.2) (layer "F.Cu") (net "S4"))
 (segment (start 150.247916 143.9) (end 150.647916 143.5) (width 0.2) (layer "F.Cu") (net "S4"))
 (segment (start 144.247916 145) (end 144.647916 145.4) (width 0.2) (layer "F.Cu") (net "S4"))
 (segment (start 153.847916 143.5) (end 154.247916 143.9) (width 0.2) (layer "F.Cu") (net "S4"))
 (segment (start 158.247916 146.1) (end 158.247916 145.4) (width 0.2) (layer "F.Cu") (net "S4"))
 (segment (start 156.647916 146.1) (end 156.647916 143.9) (width 0.2) (layer "F.Cu") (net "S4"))
 (segment (start 151.847916 143.9) (end 152.247916 143.5) (width 0.2) (layer "F.Cu") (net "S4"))
 (segment (start 155.047916 143.9) (end 155.447916 143.5) (width 0.2) (layer "F.Cu") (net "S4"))
 (segment (start 151.047916 146.1) (end 151.447916 146.5) (width 0.2) (layer "F.Cu") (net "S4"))
 (segment (start 157.847916 146.5) (end 158.247916 146.1) (width 0.2) (layer "F.Cu") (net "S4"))
 (segment (start 157.447916 143.9) (end 157.447916 146.1) (width 0.2) (layer "F.Cu") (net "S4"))
 (segment (start 157.047916 143.5) (end 157.447916 143.9) (width 0.2) (layer "F.Cu") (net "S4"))
 (segment (start 145.447916 146.1) (end 145.447916 143.9) (width 0.2) (layer "F.Cu") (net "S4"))
 (segment (start 153.447916 143.9) (end 153.847916 143.5) (width 0.2) (layer "F.Cu") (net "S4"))
 (segment (start 156.647916 143.9) (end 157.047916 143.5) (width 0.2) (layer "F.Cu") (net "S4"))
 (segment (start 144.647916 145.4) (end 144.647916 146.1) (width 0.2) (layer "F.Cu") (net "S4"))
 (segment (start 157.447916 146.1) (end 157.847916 146.5) (width 0.2) (layer "F.Cu") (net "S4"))
 (segment (start 155.447916 143.5) (end 155.847916 143.9) (width 0.2) (layer "F.Cu") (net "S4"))
 (segment (start 115 145) (end 118 148) (width 0.2) (layer "F.Cu") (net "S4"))
 (segment (start 144.647916 146.1) (end 145.047916 146.5) (width 0.2) (layer "F.Cu") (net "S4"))
 (segment (start 158.647916 145) (end 159.74056 145) (width 0.2) (layer "F.Cu") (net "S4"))
 (segment (start 150.247916 146.1) (end 150.247916 143.9) (width 0.2) (layer "F.Cu") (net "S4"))
 (segment (start 139 145) (end 144.247916 145) (width 0.2) (layer "F.Cu") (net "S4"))
 (segment (start 149.447916 143.9) (end 149.447916 146.1) (width 0.2) (layer "F.Cu") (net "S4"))
 (segment (start 118 148) (end 136 148) (width 0.2) (layer "F.Cu") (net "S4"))
 (segment (start 150.647916 143.5) (end 151.047916 143.9) (width 0.2) (layer "F.Cu") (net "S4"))
 (segment (start 151.847916 146.1) (end 151.847916 143.9) (width 0.2) (layer "F.Cu") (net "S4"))
 (segment (start 156.247916 146.5) (end 156.647916 146.1) (width 0.2) (layer "F.Cu") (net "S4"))
 (segment (start 146.247916 146.1) (end 146.647916 146.5) (width 0.2) (layer "F.Cu") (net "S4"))
 (segment (start 159.74056 145) (end 164 145) (width 0.2) (layer "F.Cu") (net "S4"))
 (segment (start 158.247916 145.4) (end 158.647916 145) (width 0.2) (layer "F.Cu") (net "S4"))
 (segment (start 153.047916 146.5) (end 153.447916 146.1) (width 0.2) (layer "F.Cu") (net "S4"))
 (segment (start 148.247916 146.5) (end 148.647916 146.1) (width 0.2) (layer "F.Cu") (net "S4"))
 (segment (start 149.047916 143.5) (end 149.447916 143.9) (width 0.2) (layer "F.Cu") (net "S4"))
 (segment (start 154.247916 146.1) (end 154.647916 146.5) (width 0.2) (layer "F.Cu") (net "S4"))
 (segment (start 154.247916 143.9) (end 154.247916 146.1) (width 0.2) (layer "F.Cu") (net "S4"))
 (segment (start 106 145) (end 115 145) (width 0.2) (layer "F.Cu") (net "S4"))
 (segment (start 151.447916 146.5) (end 151.847916 146.1) (width 0.2) (layer "F.Cu") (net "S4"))
 (segment (start 147.047916 143.9) (end 147.447916 143.5) (width 0.2) (layer "F.Cu") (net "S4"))
 (segment (start 152.247916 143.5) (end 152.647916 143.9) (width 0.2) (layer "F.Cu") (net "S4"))
 (segment (start 155.047916 146.1) (end 155.047916 143.9) (width 0.2) (layer "F.Cu") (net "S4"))
 (segment (start 147.447916 143.5) (end 147.847916 143.9) (width 0.2) (layer "F.Cu") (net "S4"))
 (segment (start 145.847916 143.5) (end 146.247916 143.9) (width 0.2) (layer "F.Cu") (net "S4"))
 (segment (start 154.647916 146.5) (end 155.047916 146.1) (width 0.2) (layer "F.Cu") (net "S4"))
 (segment (start 151.047916 143.9) (end 151.047916 146.1) (width 0.2) (layer "F.Cu") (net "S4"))
 (segment (start 152.647916 146.1) (end 153.047916 146.5) (width 0.2) (layer "F.Cu") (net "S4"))
 (segment (start 149.447916 146.1) (end 149.847916 146.5) (width 0.2) (layer "F.Cu") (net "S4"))
 (segment (start 145.047916 146.5) (end 145.447916 146.1) (width 0.2) (layer "F.Cu") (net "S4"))
 (segment (start 148.647916 143.9) (end 149.047916 143.5) (width 0.2) (layer "F.Cu") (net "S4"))
 (segment (start 147.047916 146.1) (end 147.047916 143.9) (width 0.2) (layer "F.Cu") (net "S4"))
 (segment (start 155.847916 143.9) (end 155.847916 146.1) (width 0.2) (layer "F.Cu") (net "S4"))
 (segment (start 136 148) (end 139 145) (width 0.2) (layer "F.Cu") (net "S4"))
 (segment (start 145.447916 143.9) (end 145.847916 143.5) (width 0.2) (layer "F.Cu") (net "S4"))
 (segment (start 147.847916 143.9) (end 147.847916 146.1) (width 0.2) (layer "F.Cu") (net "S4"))
 (segment (start 146.647916 146.5) (end 147.047916 146.1) (width 0.2) (layer "F.Cu") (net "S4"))
 (segment (start 155.847916 146.1) (end 156.247916 146.5) (width 0.2) (layer "F.Cu") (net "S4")))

